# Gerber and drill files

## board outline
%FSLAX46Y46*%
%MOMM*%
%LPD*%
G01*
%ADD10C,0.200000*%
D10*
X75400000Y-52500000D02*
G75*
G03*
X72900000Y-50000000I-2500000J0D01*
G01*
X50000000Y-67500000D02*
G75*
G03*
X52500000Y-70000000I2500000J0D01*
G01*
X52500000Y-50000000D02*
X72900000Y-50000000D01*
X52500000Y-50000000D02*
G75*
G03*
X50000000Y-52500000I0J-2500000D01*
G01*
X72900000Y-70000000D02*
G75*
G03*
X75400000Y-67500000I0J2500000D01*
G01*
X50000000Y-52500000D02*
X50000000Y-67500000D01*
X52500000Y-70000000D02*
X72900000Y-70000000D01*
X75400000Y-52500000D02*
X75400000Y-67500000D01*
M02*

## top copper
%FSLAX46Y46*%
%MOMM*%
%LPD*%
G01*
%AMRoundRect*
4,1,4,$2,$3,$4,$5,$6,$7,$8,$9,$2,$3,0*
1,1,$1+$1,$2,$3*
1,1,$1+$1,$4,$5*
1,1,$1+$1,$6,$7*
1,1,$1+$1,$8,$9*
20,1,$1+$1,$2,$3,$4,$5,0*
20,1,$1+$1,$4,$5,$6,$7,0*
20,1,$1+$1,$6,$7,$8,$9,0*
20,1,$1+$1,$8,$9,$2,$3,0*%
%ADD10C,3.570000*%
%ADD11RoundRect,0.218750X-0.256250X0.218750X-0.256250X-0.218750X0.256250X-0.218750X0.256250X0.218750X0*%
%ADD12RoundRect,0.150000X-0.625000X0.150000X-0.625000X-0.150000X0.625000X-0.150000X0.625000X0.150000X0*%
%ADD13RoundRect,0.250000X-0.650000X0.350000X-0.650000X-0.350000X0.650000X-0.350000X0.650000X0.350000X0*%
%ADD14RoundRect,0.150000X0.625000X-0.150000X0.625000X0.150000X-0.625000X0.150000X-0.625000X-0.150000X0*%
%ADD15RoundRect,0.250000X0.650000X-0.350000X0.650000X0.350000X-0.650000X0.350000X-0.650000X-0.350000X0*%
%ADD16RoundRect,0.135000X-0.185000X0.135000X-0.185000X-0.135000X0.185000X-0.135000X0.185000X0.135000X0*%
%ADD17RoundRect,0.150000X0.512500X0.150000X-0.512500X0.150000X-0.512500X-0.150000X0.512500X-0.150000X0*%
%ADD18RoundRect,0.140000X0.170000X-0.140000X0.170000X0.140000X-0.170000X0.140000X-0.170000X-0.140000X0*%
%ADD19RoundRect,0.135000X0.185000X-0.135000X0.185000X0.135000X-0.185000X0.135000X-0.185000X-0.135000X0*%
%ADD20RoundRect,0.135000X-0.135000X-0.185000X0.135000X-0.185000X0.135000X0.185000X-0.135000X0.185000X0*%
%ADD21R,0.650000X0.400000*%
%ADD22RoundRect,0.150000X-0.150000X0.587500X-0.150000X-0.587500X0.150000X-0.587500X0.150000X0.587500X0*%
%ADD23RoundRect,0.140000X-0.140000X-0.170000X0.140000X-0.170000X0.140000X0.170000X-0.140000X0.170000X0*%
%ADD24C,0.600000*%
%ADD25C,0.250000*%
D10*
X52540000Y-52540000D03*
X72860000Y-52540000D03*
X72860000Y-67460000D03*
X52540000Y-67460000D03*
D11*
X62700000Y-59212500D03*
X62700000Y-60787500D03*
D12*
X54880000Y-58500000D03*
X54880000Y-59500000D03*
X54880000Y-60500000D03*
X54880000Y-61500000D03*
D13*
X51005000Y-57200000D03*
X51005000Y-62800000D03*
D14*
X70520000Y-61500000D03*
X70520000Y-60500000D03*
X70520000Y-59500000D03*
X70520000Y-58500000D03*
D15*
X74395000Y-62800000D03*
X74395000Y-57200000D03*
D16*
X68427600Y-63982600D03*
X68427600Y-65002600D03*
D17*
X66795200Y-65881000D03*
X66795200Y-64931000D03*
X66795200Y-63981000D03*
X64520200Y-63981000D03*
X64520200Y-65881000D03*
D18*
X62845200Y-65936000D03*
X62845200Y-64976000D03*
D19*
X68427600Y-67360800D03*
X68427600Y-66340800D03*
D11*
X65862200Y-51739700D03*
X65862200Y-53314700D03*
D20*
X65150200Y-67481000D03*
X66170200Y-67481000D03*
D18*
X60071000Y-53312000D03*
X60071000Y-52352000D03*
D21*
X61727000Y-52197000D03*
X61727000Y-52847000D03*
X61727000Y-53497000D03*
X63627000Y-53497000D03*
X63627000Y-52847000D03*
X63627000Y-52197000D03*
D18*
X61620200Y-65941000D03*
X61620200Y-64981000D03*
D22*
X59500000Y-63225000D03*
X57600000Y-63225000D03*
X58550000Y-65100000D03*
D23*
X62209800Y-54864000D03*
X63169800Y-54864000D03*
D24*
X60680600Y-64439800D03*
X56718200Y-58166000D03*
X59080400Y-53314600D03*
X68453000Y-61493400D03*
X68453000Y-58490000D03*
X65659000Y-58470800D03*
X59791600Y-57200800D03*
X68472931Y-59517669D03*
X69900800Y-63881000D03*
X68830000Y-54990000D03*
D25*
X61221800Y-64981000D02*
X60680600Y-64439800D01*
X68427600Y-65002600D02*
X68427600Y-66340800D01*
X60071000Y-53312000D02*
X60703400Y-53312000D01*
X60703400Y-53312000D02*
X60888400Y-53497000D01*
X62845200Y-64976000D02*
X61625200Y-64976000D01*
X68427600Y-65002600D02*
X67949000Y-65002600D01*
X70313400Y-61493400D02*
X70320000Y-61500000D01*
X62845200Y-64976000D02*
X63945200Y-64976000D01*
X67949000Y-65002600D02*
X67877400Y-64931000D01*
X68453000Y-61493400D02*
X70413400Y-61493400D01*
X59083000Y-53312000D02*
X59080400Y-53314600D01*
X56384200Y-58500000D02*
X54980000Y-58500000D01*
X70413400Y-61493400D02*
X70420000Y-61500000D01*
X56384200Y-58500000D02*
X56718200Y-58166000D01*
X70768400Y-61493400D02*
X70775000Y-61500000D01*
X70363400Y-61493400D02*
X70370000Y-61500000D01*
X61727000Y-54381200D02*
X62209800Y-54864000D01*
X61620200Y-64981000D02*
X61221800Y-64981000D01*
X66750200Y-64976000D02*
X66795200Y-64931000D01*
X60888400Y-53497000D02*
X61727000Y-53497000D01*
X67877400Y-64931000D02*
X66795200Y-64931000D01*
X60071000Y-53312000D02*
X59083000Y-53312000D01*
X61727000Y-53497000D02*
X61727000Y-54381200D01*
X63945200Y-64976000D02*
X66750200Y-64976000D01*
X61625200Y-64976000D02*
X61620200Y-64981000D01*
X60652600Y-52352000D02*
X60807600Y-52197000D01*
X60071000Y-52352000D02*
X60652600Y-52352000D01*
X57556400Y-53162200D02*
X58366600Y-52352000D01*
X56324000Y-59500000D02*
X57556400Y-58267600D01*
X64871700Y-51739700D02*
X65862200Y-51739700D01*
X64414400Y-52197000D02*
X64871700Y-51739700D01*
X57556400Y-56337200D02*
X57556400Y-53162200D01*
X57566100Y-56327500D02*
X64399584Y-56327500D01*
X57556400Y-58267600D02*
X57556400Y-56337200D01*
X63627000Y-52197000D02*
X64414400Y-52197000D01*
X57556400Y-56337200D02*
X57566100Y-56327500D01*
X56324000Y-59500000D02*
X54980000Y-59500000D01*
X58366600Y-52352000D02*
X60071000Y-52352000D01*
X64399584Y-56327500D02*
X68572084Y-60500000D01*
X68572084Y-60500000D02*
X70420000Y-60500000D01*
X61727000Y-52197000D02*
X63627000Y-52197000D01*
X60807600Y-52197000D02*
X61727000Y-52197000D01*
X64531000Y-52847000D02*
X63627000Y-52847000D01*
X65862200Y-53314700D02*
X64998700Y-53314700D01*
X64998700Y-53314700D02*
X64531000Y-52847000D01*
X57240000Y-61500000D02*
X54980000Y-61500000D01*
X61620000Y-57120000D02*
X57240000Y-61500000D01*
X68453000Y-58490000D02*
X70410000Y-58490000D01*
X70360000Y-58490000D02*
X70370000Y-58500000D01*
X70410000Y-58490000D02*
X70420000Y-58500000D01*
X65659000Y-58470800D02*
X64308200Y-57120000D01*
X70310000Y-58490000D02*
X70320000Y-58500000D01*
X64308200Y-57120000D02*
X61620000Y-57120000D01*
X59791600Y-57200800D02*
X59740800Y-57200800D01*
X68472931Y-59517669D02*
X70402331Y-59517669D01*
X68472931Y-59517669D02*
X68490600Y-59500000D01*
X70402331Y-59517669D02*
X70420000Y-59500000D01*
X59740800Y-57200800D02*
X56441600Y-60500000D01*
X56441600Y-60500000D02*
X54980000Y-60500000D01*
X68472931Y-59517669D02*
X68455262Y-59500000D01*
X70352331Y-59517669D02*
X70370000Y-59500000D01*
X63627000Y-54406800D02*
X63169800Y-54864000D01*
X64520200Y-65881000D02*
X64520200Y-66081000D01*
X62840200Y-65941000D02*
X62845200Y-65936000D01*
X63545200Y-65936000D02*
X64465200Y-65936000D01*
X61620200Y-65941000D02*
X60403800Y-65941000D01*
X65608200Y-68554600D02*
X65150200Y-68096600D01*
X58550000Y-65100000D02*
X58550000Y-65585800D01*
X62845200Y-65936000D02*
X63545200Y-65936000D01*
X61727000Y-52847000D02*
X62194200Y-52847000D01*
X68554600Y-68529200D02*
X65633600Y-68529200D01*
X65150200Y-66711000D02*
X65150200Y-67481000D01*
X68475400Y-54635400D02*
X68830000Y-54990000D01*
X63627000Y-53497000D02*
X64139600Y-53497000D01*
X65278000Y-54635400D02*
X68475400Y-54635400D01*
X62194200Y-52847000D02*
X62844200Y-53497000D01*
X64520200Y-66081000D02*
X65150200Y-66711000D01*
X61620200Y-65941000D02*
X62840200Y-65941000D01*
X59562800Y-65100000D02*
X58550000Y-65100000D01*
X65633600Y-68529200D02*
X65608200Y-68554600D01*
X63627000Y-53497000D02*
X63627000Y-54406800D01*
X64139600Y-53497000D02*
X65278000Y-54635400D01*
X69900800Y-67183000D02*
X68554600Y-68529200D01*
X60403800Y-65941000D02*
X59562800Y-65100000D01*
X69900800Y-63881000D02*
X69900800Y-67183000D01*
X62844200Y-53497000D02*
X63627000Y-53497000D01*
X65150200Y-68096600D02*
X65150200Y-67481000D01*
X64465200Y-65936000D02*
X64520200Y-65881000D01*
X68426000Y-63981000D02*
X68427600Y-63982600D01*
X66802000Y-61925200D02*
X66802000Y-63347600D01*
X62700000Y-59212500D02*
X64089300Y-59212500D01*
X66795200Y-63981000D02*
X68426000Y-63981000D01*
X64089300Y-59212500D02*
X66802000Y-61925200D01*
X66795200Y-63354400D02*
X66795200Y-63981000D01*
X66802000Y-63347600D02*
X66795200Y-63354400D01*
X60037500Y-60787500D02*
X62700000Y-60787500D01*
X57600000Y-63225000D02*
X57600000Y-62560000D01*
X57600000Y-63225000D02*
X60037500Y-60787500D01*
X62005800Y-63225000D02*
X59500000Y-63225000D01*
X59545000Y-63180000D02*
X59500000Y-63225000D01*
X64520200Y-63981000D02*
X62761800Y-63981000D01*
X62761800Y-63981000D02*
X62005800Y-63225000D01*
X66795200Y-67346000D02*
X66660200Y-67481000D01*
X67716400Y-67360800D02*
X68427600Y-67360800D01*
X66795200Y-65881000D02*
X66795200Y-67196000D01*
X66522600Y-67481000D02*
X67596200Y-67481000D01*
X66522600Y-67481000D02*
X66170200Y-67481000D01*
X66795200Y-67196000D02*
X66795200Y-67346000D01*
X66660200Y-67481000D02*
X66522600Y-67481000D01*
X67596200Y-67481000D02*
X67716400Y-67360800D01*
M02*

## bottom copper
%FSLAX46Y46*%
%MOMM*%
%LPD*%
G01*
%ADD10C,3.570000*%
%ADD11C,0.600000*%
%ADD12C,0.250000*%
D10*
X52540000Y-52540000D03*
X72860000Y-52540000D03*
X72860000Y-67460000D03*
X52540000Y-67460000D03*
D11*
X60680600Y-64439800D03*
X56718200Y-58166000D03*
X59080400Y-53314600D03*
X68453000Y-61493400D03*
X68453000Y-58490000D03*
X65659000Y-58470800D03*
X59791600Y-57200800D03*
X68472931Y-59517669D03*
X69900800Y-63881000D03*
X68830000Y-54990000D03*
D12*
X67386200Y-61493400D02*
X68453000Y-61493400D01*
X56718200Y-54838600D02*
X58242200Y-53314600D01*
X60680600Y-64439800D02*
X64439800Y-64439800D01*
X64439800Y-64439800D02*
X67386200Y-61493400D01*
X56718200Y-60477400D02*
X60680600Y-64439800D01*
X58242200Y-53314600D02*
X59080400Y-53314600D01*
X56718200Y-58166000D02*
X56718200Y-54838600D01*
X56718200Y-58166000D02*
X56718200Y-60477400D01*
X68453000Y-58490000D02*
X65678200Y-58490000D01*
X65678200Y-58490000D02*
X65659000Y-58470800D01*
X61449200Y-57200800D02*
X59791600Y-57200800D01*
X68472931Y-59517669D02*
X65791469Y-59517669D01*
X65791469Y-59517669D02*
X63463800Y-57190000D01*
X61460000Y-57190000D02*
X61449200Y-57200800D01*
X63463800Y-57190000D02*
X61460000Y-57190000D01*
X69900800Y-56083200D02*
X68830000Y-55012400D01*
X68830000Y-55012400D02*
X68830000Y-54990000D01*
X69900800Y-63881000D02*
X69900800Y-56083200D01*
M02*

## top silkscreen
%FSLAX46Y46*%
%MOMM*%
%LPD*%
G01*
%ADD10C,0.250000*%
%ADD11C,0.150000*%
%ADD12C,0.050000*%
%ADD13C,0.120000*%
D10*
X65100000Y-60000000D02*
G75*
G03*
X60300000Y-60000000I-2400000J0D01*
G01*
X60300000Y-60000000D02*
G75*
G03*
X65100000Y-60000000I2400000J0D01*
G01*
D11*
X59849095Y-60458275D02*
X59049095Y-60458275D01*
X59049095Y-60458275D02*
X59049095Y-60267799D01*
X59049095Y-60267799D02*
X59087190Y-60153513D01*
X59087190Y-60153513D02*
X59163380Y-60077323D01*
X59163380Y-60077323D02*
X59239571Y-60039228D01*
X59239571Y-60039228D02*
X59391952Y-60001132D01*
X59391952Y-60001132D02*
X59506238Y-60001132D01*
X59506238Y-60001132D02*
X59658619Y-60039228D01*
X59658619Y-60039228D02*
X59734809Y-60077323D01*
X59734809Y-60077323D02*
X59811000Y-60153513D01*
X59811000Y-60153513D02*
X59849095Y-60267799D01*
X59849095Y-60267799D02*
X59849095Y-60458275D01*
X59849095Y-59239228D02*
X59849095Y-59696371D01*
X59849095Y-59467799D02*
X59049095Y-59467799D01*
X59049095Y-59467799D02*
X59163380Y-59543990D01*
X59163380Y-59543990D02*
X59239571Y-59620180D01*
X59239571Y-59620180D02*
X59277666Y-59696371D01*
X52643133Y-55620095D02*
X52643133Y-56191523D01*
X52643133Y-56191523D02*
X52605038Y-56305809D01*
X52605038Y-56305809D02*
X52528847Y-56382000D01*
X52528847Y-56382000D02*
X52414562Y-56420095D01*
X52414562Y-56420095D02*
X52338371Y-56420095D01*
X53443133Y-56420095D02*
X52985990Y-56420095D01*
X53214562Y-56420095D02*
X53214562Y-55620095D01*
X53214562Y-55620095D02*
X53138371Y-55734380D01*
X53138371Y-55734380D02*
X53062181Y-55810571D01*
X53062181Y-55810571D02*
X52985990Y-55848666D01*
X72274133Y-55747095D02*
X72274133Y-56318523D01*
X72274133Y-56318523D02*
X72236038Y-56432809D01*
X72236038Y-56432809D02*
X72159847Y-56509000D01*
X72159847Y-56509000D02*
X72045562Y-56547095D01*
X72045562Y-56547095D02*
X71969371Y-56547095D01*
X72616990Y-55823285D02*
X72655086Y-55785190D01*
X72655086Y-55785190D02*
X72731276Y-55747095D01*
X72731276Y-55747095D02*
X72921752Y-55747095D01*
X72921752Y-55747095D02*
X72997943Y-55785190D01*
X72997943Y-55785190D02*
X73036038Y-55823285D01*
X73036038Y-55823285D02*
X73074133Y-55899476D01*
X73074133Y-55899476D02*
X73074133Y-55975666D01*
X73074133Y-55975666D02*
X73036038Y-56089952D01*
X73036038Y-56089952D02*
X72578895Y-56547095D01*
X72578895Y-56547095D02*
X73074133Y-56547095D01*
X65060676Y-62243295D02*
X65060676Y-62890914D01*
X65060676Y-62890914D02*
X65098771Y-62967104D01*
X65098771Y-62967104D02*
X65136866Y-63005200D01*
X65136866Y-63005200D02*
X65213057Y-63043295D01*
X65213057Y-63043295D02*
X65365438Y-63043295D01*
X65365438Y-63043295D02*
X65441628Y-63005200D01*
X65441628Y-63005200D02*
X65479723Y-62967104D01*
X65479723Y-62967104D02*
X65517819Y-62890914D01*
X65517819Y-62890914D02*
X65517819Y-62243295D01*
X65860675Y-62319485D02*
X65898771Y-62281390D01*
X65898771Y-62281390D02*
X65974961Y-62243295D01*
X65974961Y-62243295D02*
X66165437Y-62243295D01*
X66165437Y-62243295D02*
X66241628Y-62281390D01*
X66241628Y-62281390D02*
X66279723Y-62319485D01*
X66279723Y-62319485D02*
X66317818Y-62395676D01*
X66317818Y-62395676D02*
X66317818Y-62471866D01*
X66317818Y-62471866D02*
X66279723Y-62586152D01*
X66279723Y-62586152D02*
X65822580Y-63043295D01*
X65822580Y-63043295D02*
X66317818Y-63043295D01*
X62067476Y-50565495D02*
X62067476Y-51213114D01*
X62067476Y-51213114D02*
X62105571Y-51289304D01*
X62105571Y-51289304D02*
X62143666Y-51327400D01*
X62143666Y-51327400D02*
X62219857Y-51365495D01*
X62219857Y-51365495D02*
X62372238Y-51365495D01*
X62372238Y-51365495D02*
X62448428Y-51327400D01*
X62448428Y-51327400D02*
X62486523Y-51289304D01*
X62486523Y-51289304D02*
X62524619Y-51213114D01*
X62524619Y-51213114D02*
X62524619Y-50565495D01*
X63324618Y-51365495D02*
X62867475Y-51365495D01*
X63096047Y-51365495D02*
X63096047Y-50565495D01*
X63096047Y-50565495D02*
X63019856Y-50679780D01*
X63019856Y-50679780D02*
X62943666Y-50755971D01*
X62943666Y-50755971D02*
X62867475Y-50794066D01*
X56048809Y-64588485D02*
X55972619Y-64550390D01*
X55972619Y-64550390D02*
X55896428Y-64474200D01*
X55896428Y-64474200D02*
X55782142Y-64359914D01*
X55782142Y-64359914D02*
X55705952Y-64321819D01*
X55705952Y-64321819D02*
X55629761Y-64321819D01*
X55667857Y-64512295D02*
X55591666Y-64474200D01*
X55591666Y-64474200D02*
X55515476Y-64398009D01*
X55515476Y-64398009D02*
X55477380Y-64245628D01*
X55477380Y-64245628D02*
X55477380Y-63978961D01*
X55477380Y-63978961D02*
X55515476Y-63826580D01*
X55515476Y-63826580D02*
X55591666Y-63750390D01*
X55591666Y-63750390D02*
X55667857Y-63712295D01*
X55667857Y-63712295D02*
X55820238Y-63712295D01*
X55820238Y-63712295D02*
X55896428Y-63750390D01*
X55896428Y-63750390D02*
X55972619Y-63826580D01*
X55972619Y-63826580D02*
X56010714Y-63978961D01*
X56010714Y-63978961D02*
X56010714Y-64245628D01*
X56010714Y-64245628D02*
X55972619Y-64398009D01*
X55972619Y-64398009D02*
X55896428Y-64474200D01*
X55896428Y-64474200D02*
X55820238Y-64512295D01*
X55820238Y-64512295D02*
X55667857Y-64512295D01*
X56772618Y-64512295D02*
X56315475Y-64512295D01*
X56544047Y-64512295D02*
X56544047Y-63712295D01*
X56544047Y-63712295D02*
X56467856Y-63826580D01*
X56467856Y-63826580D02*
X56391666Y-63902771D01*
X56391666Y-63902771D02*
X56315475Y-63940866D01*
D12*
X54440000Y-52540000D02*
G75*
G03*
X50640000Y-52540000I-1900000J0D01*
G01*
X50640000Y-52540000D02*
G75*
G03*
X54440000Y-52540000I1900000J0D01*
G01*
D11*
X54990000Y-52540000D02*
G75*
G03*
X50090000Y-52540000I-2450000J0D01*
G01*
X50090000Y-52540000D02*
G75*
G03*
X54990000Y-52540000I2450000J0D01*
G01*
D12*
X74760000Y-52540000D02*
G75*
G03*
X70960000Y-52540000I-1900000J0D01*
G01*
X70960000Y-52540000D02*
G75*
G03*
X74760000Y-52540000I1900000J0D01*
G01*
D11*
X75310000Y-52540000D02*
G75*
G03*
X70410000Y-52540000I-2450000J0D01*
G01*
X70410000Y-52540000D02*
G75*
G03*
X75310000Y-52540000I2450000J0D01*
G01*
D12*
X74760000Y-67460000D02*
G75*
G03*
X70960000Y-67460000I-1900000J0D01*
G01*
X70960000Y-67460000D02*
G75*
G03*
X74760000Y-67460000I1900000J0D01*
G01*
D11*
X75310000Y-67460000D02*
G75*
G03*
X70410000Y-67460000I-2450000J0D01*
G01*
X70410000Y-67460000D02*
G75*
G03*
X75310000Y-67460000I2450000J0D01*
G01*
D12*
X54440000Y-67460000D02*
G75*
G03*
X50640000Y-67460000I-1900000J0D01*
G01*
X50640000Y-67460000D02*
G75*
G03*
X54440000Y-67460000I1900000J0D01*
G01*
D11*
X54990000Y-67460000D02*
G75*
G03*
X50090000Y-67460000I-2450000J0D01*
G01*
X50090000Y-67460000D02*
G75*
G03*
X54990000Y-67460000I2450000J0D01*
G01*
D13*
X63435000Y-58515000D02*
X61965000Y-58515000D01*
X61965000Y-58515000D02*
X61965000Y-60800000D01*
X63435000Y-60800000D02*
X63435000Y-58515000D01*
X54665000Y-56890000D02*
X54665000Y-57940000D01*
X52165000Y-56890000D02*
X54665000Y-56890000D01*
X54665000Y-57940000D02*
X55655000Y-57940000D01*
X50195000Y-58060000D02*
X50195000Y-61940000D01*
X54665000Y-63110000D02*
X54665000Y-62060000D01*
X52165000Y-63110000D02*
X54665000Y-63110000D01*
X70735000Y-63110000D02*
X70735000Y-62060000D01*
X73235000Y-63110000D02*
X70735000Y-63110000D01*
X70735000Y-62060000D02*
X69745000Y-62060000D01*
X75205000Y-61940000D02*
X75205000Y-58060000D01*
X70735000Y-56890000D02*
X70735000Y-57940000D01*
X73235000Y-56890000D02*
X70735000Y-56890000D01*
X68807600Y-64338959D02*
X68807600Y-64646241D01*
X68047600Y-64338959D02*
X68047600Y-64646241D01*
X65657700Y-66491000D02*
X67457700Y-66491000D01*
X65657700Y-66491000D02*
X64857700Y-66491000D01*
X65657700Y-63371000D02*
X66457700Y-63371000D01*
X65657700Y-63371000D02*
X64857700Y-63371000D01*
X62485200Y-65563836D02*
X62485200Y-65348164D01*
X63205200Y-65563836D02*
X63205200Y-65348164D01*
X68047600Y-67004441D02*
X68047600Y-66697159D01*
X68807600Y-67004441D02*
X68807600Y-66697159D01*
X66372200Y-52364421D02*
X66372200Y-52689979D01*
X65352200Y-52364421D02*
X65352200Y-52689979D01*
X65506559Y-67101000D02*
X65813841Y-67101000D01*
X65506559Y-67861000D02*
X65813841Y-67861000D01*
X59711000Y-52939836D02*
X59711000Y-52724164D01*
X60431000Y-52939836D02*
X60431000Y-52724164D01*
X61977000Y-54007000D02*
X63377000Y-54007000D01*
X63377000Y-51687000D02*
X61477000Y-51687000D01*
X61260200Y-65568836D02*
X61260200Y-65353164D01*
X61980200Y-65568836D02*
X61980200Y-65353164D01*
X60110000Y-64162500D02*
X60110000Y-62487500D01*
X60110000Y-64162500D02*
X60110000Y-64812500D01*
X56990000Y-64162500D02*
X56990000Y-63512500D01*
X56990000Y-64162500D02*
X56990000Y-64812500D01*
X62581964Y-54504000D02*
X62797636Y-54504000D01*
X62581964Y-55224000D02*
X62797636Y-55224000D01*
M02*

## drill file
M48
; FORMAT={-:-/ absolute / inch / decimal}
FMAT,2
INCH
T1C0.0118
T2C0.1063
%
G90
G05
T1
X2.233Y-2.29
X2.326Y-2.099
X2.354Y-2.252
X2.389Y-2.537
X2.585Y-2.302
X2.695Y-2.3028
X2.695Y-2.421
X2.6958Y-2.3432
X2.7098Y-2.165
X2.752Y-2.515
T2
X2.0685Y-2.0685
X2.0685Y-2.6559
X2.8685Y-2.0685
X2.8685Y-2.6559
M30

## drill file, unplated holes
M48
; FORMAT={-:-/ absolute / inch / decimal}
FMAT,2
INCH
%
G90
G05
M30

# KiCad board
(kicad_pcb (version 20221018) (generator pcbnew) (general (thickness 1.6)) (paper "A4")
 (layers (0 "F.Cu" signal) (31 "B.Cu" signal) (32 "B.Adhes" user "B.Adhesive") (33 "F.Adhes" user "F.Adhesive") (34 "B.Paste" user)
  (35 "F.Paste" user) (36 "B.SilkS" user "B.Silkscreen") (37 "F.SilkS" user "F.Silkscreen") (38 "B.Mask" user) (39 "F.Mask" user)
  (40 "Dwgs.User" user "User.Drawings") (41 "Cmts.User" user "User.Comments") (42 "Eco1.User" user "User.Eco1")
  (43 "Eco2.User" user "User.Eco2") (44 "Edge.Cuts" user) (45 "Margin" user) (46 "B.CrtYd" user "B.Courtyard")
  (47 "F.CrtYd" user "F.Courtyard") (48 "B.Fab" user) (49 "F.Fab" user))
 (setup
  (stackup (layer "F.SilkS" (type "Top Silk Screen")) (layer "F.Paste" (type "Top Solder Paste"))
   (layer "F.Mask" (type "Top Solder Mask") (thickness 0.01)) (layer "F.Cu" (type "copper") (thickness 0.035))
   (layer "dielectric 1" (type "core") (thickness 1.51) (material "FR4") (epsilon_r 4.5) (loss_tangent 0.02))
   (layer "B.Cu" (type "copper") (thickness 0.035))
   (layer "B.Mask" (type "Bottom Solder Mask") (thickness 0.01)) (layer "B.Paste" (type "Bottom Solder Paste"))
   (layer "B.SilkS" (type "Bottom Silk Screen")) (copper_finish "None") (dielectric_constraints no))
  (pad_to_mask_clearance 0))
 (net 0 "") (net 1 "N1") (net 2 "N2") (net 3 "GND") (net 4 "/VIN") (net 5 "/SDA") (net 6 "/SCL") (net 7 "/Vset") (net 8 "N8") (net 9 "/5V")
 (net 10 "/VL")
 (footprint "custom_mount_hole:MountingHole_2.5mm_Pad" (layer "F.Cu") (at 52.54 52.54)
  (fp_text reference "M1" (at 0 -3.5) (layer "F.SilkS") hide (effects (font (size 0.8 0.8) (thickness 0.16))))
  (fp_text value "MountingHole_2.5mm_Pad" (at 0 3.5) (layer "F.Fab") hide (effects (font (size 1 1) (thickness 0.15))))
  (fp_circle (center 0 0) (end 1.9 0) (stroke (width 0.05) (type solid)) (fill none) (layer "F.SilkS"))
  (fp_circle (center 0 0) (end 2.45 0) (stroke (width 0.15) (type solid)) (fill none) (layer "F.SilkS"))
  (pad "~" thru_hole circle (at 0 0) (size 3.57 3.57) (drill 2.7) (layers "*.Cu" "*.Mask")))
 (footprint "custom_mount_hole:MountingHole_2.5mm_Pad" (layer "F.Cu") (at 72.86 52.54)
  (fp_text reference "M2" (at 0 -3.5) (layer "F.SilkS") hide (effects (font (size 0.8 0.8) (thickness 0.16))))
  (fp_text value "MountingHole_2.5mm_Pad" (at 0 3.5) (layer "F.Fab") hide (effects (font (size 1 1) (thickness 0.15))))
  (fp_circle (center 0 0) (end 1.9 0) (stroke (width 0.05) (type solid)) (fill none) (layer "F.SilkS"))
  (fp_circle (center 0 0) (end 2.45 0) (stroke (width 0.15) (type solid)) (fill none) (layer "F.SilkS"))
  (pad "~" thru_hole circle (at 0 0) (size 3.57 3.57) (drill 2.7) (layers "*.Cu" "*.Mask")))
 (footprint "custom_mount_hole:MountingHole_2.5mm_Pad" (layer "F.Cu") (at 72.86 67.46)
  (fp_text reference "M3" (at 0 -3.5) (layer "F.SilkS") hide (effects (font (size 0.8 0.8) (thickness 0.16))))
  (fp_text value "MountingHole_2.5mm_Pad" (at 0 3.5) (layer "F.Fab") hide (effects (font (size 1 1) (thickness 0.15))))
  (fp_circle (center 0 0) (end 1.9 0) (stroke (width 0.05) (type solid)) (fill none) (layer "F.SilkS"))
  (fp_circle (center 0 0) (end 2.45 0) (stroke (width 0.15) (type solid)) (fill none) (layer "F.SilkS"))
  (pad "~" thru_hole circle (at 0 0) (size 3.57 3.57) (drill 2.7) (layers "*.Cu" "*.Mask")))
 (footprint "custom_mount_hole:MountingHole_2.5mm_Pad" (layer "F.Cu") (at 52.54 67.46)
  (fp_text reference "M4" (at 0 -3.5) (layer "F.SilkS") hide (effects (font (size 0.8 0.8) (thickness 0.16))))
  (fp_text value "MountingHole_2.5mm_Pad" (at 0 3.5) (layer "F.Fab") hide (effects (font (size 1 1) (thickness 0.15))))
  (fp_circle (center 0 0) (end 1.9 0) (stroke (width 0.05) (type solid)) (fill none) (layer "F.SilkS"))
  (fp_circle (center 0 0) (end 2.45 0) (stroke (width 0.15) (type solid)) (fill none) (layer "F.SilkS"))
  (pad "~" thru_hole circle (at 0 0) (size 3.57 3.57) (drill 2.7) (layers "*.Cu" "*.Mask")))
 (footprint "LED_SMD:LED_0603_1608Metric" (layer "F.Cu") (at 62.7 60 -90)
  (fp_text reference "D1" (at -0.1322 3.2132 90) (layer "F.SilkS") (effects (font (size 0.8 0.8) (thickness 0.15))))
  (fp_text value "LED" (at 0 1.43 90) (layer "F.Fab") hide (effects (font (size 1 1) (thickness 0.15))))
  (fp_line (start -1.485 -0.735) (end -1.485 0.735) (stroke (width 0.12) (type solid)) (layer "F.SilkS"))
  (fp_line (start -1.485 0.735) (end 0.8 0.735) (stroke (width 0.12) (type solid)) (layer "F.SilkS"))
  (fp_line (start 0.8 -0.735) (end -1.485 -0.735) (stroke (width 0.12) (type solid)) (layer "F.SilkS"))
  (pad "1" smd roundrect (at -0.7875 0 270) (size 0.875 0.95) (layers "F.Cu" "F.Paste" "F.Mask") (roundrect_rratio 0.25) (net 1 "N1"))
  (pad "2" smd roundrect (at 0.7875 0 270) (size 0.875 0.95) (layers "F.Cu" "F.Paste" "F.Mask") (roundrect_rratio 0.25) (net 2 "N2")))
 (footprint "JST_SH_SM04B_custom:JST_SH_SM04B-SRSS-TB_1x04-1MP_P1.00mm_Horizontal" (layer "F.Cu") (at 52.88 60 -90)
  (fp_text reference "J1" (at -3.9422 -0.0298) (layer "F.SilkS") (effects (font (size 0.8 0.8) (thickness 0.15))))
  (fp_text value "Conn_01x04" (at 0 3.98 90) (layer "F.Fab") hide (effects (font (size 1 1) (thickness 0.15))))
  (fp_line (start -3.11 -1.785) (end -2.06 -1.785) (stroke (width 0.12) (type solid)) (layer "F.SilkS"))
  (fp_line (start -3.11 0.715) (end -3.11 -1.785) (stroke (width 0.12) (type solid)) (layer "F.SilkS"))
  (fp_line (start -2.06 -1.785) (end -2.06 -2.775) (stroke (width 0.12) (type solid)) (layer "F.SilkS"))
  (fp_line (start -1.94 2.685) (end 1.94 2.685) (stroke (width 0.12) (type solid)) (layer "F.SilkS"))
  (fp_line (start 3.11 -1.785) (end 2.06 -1.785) (stroke (width 0.12) (type solid)) (layer "F.SilkS"))
  (fp_line (start 3.11 0.715) (end 3.11 -1.785) (stroke (width 0.12) (type solid)) (layer "F.SilkS"))
  (pad "1" smd roundrect (at -1.5 -2 270) (size 0.6 1.55) (layers "F.Cu" "F.Paste" "F.Mask") (roundrect_rratio 0.25) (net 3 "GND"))
  (pad "2" smd roundrect (at -0.5 -2 270) (size 0.6 1.55) (layers "F.Cu" "F.Paste" "F.Mask") (roundrect_rratio 0.25) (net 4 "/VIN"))
  (pad "3" smd roundrect (at 0.5 -2 270) (size 0.6 1.55) (layers "F.Cu" "F.Paste" "F.Mask") (roundrect_rratio 0.25) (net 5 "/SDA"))
  (pad "4" smd roundrect (at 1.5 -2 270) (size 0.6 1.55) (layers "F.Cu" "F.Paste" "F.Mask") (roundrect_rratio 0.25) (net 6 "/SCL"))
  (pad "MP" smd roundrect (at -2.8 1.875 270) (size 1.2 1.8) (layers "F.Cu" "F.Paste" "F.Mask") (roundrect_rratio 0.2083333333))
  (pad "MP" smd roundrect (at 2.8 1.875 270) (size 1.2 1.8) (layers "F.Cu" "F.Paste" "F.Mask") (roundrect_rratio 0.2083333333)))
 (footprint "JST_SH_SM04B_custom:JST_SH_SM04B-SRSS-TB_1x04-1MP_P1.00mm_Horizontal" (layer "F.Cu") (at 72.52 60 90)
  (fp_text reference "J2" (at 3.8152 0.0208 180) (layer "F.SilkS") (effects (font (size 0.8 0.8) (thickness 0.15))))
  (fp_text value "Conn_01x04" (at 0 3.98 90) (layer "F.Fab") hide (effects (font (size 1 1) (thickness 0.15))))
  (fp_line (start -3.11 -1.785) (end -2.06 -1.785) (stroke (width 0.12) (type solid)) (layer "F.SilkS"))
  (fp_line (start -3.11 0.715) (end -3.11 -1.785) (stroke (width 0.12) (type solid)) (layer "F.SilkS"))
  (fp_line (start -2.06 -1.785) (end -2.06 -2.775) (stroke (width 0.12) (type solid)) (layer "F.SilkS"))
  (fp_line (start -1.94 2.685) (end 1.94 2.685) (stroke (width 0.12) (type solid)) (layer "F.SilkS"))
  (fp_line (start 3.11 -1.785) (end 2.06 -1.785) (stroke (width 0.12) (type solid)) (layer "F.SilkS"))
  (fp_line (start 3.11 0.715) (end 3.11 -1.785) (stroke (width 0.12) (type solid)) (layer "F.SilkS"))
  (pad "1" smd roundrect (at -1.5 -2 90) (size 0.6 1.55) (layers "F.Cu" "F.Paste" "F.Mask") (roundrect_rratio 0.25) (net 3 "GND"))
  (pad "2" smd roundrect (at -0.5 -2 90) (size 0.6 1.55) (layers "F.Cu" "F.Paste" "F.Mask") (roundrect_rratio 0.25) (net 4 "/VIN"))
  (pad "3" smd roundrect (at 0.5 -2 90) (size 0.6 1.55) (layers "F.Cu" "F.Paste" "F.Mask") (roundrect_rratio 0.25) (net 5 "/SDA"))
  (pad "4" smd roundrect (at 1.5 -2 90) (size 0.6 1.55) (layers "F.Cu" "F.Paste" "F.Mask") (roundrect_rratio 0.25) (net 6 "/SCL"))
  (pad "MP" smd roundrect (at -2.8 1.875 90) (size 1.2 1.8) (layers "F.Cu" "F.Paste" "F.Mask") (roundrect_rratio 0.2083333333))
  (pad "MP" smd roundrect (at 2.8 1.875 90) (size 1.2 1.8) (layers "F.Cu" "F.Paste" "F.Mask") (roundrect_rratio 0.2083333333)))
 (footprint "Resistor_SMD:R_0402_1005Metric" (layer "F.Cu") (at 68.4276 64.4926 -90)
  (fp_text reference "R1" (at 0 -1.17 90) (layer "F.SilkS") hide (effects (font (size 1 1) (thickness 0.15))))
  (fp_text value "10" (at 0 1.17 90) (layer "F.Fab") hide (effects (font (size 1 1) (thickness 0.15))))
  (fp_line (start -0.153641 -0.38) (end 0.153641 -0.38) (stroke (width 0.12) (type solid)) (layer "F.SilkS"))
  (fp_line (start -0.153641 0.38) (end 0.153641 0.38) (stroke (width 0.12) (type solid)) (layer "F.SilkS"))
  (pad "1" smd roundrect (at -0.51 0 270) (size 0.54 0.64) (layers "F.Cu" "F.Paste" "F.Mask") (roundrect_rratio 0.25) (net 1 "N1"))
  (pad "2" smd roundrect (at 0.51 0 270) (size 0.54 0.64) (layers "F.Cu" "F.Paste" "F.Mask") (roundrect_rratio 0.25) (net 3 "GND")))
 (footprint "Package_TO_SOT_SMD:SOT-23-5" (layer "F.Cu") (at 65.6577 64.931 180)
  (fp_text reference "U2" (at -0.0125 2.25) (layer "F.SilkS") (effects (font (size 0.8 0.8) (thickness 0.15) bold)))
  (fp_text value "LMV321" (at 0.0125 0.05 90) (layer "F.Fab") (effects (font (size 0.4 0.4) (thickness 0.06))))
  (fp_line (start 0 -1.56) (end -1.8 -1.56) (stroke (width 0.12) (type solid)) (layer "F.SilkS"))
  (fp_line (start 0 -1.56) (end 0.8 -1.56) (stroke (width 0.12) (type solid)) (layer "F.SilkS"))
  (fp_line (start 0 1.56) (end -0.8 1.56) (stroke (width 0.12) (type solid)) (layer "F.SilkS"))
  (fp_line (start 0 1.56) (end 0.8 1.56) (stroke (width 0.12) (type solid)) (layer "F.SilkS"))
  (pad "1" smd roundrect (at -1.1375 -0.95 180) (size 1.325 0.6) (layers "F.Cu" "F.Paste" "F.Mask") (roundrect_rratio 0.25) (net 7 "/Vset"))
  (pad "2" smd roundrect (at -1.1375 0 180) (size 1.325 0.6) (layers "F.Cu" "F.Paste" "F.Mask") (roundrect_rratio 0.25) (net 3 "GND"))
  (pad "3" smd roundrect (at -1.1375 0.95 180) (size 1.325 0.6) (layers "F.Cu" "F.Paste" "F.Mask") (roundrect_rratio 0.25) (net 1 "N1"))
  (pad "4" smd roundrect (at 1.1375 0.95 180) (size 1.325 0.6) (layers "F.Cu" "F.Paste" "F.Mask") (roundrect_rratio 0.25) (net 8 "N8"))
  (pad "5" smd roundrect (at 1.1375 -0.95 180) (size 1.325 0.6) (layers "F.Cu" "F.Paste" "F.Mask") (roundrect_rratio 0.25) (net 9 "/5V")))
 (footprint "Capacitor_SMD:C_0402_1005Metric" (layer "F.Cu") (at 62.8452 65.456 90)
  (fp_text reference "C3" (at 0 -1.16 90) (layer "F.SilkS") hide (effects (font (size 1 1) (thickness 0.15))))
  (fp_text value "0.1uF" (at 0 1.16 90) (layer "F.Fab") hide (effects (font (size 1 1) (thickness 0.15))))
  (fp_line (start -0.107836 -0.36) (end 0.107836 -0.36) (stroke (width 0.12) (type solid)) (layer "F.SilkS"))
  (fp_line (start -0.107836 0.36) (end 0.107836 0.36) (stroke (width 0.12) (type solid)) (layer "F.SilkS"))
  (pad "1" smd roundrect (at -0.48 0 90) (size 0.56 0.62) (layers "F.Cu" "F.Paste" "F.Mask") (roundrect_rratio 0.25) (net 9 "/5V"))
  (pad "2" smd roundrect (at 0.48 0 90) (size 0.56 0.62) (layers "F.Cu" "F.Paste" "F.Mask") (roundrect_rratio 0.25) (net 3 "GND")))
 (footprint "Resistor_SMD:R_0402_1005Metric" (layer "F.Cu") (at 68.4276 66.8508 90)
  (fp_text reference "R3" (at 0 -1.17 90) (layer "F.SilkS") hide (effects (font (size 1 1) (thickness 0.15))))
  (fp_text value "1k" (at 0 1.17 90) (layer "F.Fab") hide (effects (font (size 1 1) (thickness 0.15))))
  (fp_line (start -0.153641 -0.38) (end 0.153641 -0.38) (stroke (width 0.12) (type solid)) (layer "F.SilkS"))
  (fp_line (start -0.153641 0.38) (end 0.153641 0.38) (stroke (width 0.12) (type solid)) (layer "F.SilkS"))
  (pad "1" smd roundrect (at -0.51 0 90) (size 0.54 0.64) (layers "F.Cu" "F.Paste" "F.Mask") (roundrect_rratio 0.25) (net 7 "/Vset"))
  (pad "2" smd roundrect (at 0.51 0 90) (size 0.54 0.64) (layers "F.Cu" "F.Paste" "F.Mask") (roundrect_rratio 0.25) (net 3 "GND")))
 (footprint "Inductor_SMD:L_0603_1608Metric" (layer "F.Cu") (at 65.8622 52.5272 -90)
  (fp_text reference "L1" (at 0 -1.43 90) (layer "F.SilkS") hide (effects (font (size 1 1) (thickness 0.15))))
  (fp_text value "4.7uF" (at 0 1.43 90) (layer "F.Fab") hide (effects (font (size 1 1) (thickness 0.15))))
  (fp_line (start -0.162779 -0.51) (end 0.162779 -0.51) (stroke (width 0.12) (type solid)) (layer "F.SilkS"))
  (fp_line (start -0.162779 0.51) (end 0.162779 0.51) (stroke (width 0.12) (type solid)) (layer "F.SilkS"))
  (pad "1" smd roundrect (at -0.7875 0 270) (size 0.875 0.95) (layers "F.Cu" "F.Paste" "F.Mask") (roundrect_rratio 0.25) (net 4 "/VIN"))
  (pad "2" smd roundrect (at 0.7875 0 270) (size 0.875 0.95) (layers "F.Cu" "F.Paste" "F.Mask") (roundrect_rratio 0.25) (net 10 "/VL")))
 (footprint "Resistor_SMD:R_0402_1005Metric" (layer "F.Cu") (at 65.6602 67.481)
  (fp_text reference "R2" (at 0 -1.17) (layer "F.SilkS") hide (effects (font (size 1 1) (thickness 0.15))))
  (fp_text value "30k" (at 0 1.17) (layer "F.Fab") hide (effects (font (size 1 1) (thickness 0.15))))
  (fp_line (start -0.153641 -0.38) (end 0.153641 -0.38) (stroke (width 0.12) (type solid)) (layer "F.SilkS"))
  (fp_line (start -0.153641 0.38) (end 0.153641 0.38) (stroke (width 0.12) (type solid)) (layer "F.SilkS"))
  (pad "1" smd roundrect (at -0.51 0) (size 0.54 0.64) (layers "F.Cu" "F.Paste" "F.Mask") (roundrect_rratio 0.25) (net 9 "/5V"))
  (pad "2" smd roundrect (at 0.51 0) (size 0.54 0.64) (layers "F.Cu" "F.Paste" "F.Mask") (roundrect_rratio 0.25) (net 7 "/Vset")))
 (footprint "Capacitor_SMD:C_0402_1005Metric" (layer "F.Cu") (at 60.071 52.832 90)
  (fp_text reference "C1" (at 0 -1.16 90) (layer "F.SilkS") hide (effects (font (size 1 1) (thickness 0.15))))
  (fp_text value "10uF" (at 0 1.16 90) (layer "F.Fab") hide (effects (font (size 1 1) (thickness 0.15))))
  (fp_line (start -0.107836 -0.36) (end 0.107836 -0.36) (stroke (width 0.12) (type solid)) (layer "F.SilkS"))
  (fp_line (start -0.107836 0.36) (end 0.107836 0.36) (stroke (width 0.12) (type solid)) (layer "F.SilkS"))
  (pad "1" smd roundrect (at -0.48 0 90) (size 0.56 0.62) (layers "F.Cu" "F.Paste" "F.Mask") (roundrect_rratio 0.25) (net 3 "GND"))
  (pad "2" smd roundrect (at 0.48 0 90) (size 0.56 0.62) (layers "F.Cu" "F.Paste" "F.Mask") (roundrect_rratio 0.25) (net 4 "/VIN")))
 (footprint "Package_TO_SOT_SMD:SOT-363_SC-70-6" (layer "F.Cu") (at 62.677 52.847)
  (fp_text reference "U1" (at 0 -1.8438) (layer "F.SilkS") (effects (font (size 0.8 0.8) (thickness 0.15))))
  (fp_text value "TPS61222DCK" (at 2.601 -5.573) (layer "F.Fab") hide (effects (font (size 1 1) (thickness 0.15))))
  (fp_line (start -0.7 1.16) (end 0.7 1.16) (stroke (width 0.12) (type solid)) (layer "F.SilkS"))
  (fp_line (start 0.7 -1.16) (end -1.2 -1.16) (stroke (width 0.12) (type solid)) (layer "F.SilkS"))
  (pad "1" smd rect (at -0.95 -0.65) (size 0.65 0.4) (layers "F.Cu" "F.Paste" "F.Mask") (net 4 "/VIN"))
  (pad "2" smd rect (at -0.95 0) (size 0.65 0.4) (layers "F.Cu" "F.Paste" "F.Mask") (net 9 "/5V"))
  (pad "3" smd rect (at -0.95 0.65) (size 0.65 0.4) (layers "F.Cu" "F.Paste" "F.Mask") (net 3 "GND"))
  (pad "4" smd rect (at 0.95 0.65) (size 0.65 0.4) (layers "F.Cu" "F.Paste" "F.Mask") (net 9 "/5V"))
  (pad "5" smd rect (at 0.95 0) (size 0.65 0.4) (layers "F.Cu" "F.Paste" "F.Mask") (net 10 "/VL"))
  (pad "6" smd rect (at 0.95 -0.65) (size 0.65 0.4) (layers "F.Cu" "F.Paste" "F.Mask") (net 4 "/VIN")))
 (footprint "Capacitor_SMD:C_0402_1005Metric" (layer "F.Cu") (at 61.6202 65.461 90)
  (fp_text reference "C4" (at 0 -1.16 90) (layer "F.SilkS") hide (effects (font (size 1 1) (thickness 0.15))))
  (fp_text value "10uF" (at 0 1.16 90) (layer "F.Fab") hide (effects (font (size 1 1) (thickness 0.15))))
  (fp_line (start -0.107836 -0.36) (end 0.107836 -0.36) (stroke (width 0.12) (type solid)) (layer "F.SilkS"))
  (fp_line (start -0.107836 0.36) (end 0.107836 0.36) (stroke (width 0.12) (type solid)) (layer "F.SilkS"))
  (pad "1" smd roundrect (at -0.48 0 90) (size 0.56 0.62) (layers "F.Cu" "F.Paste" "F.Mask") (roundrect_rratio 0.25) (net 9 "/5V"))
  (pad "2" smd roundrect (at 0.48 0 90) (size 0.56 0.62) (layers "F.Cu" "F.Paste" "F.Mask") (roundrect_rratio 0.25) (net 3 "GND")))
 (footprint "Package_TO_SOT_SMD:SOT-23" (layer "F.Cu") (at 58.55 64.1625 -90)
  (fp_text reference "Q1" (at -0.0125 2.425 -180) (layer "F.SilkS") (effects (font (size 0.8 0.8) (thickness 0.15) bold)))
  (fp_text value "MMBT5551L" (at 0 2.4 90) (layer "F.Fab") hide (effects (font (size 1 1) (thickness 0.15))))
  (fp_line (start 0 -1.56) (end -1.675 -1.56) (stroke (width 0.12) (type solid)) (layer "F.SilkS"))
  (fp_line (start 0 -1.56) (end 0.65 -1.56) (stroke (width 0.12) (type solid)) (layer "F.SilkS"))
  (fp_line (start 0 1.56) (end -0.65 1.56) (stroke (width 0.12) (type solid)) (layer "F.SilkS"))
  (fp_line (start 0 1.56) (end 0.65 1.56) (stroke (width 0.12) (type solid)) (layer "F.SilkS"))
  (pad "1" smd roundrect (at -0.9375 -0.95 270) (size 1.475 0.6) (layers "F.Cu" "F.Paste" "F.Mask") (roundrect_rratio 0.25) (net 8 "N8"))
  (pad "2" smd roundrect (at -0.9375 0.95 270) (size 1.475 0.6) (layers "F.Cu" "F.Paste" "F.Mask") (roundrect_rratio 0.25) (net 2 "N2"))
  (pad "3" smd roundrect (at 0.9375 0 270) (size 1.475 0.6) (layers "F.Cu" "F.Paste" "F.Mask") (roundrect_rratio 0.25) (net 9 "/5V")))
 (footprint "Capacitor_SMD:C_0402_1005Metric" (layer "F.Cu") (at 62.6898 54.864)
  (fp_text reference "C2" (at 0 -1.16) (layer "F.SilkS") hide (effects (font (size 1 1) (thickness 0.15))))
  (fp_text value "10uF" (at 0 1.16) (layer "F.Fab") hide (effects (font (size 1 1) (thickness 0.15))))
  (fp_line (start -0.107836 -0.36) (end 0.107836 -0.36) (stroke (width 0.12) (type solid)) (layer "F.SilkS"))
  (fp_line (start -0.107836 0.36) (end 0.107836 0.36) (stroke (width 0.12) (type solid)) (layer "F.SilkS"))
  (pad "1" smd roundrect (at -0.48 0) (size 0.56 0.62) (layers "F.Cu" "F.Paste" "F.Mask") (roundrect_rratio 0.25) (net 3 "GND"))
  (pad "2" smd roundrect (at 0.48 0) (size 0.56 0.62) (layers "F.Cu" "F.Paste" "F.Mask") (roundrect_rratio 0.25) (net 9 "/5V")))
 (gr_circle (center 62.7 60) (end 65.1 60) (stroke (width 0.25) (type solid)) (fill none) (layer "F.SilkS"))
 (gr_arc (start 72.9 50) (mid 74.667767 50.732233) (end 75.4 52.5) (stroke (width 0.2) (type solid)) (layer "Edge.Cuts"))
 (gr_arc (start 52.5 70) (mid 50.732233 69.267767) (end 50 67.5) (stroke (width 0.2) (type solid)) (layer "Edge.Cuts"))
 (gr_line (start 52.5 50) (end 72.9 50) (stroke (width 0.2) (type solid)) (layer "Edge.Cuts"))
 (gr_arc (start 50 52.5) (mid 50.732233 50.732233) (end 52.5 50) (stroke (width 0.2) (type solid)) (layer "Edge.Cuts"))
 (gr_arc (start 75.4 67.5) (mid 74.667767 69.267767) (end 72.9 70) (stroke (width 0.2) (type solid)) (layer "Edge.Cuts"))
 (gr_line (start 50 52.5) (end 50 67.5) (stroke (width 0.2) (type solid)) (layer "Edge.Cuts"))
 (gr_line (start 52.5 70) (end 72.9 70) (stroke (width 0.2) (type solid)) (layer "Edge.Cuts"))
 (gr_line (start 75.4 52.5) (end 75.4 67.5) (stroke (width 0.2) (type solid)) (layer "Edge.Cuts"))
 (segment (start 61.2218 64.981) (end 60.6806 64.4398) (width 0.25) (layer "F.Cu") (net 3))
 (segment (start 68.4276 65.0026) (end 68.4276 66.3408) (width 0.25) (layer "F.Cu") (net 3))
 (segment (start 60.071 53.312) (end 60.7034 53.312) (width 0.25) (layer "F.Cu") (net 3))
 (segment (start 60.7034 53.312) (end 60.8884 53.497) (width 0.25) (layer "F.Cu") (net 3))
 (segment (start 62.8452 64.976) (end 61.6252 64.976) (width 0.25) (layer "F.Cu") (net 3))
 (segment (start 68.4276 65.0026) (end 67.949 65.0026) (width 0.25) (layer "F.Cu") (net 3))
 (segment (start 70.3134 61.4934) (end 70.32 61.5) (width 0.25) (layer "F.Cu") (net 3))
 (segment (start 62.8452 64.976) (end 63.9452 64.976) (width 0.25) (layer "F.Cu") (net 3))
 (segment (start 67.949 65.0026) (end 67.8774 64.931) (width 0.25) (layer "F.Cu") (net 3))
 (segment (start 68.453 61.4934) (end 70.4134 61.4934) (width 0.25) (layer "F.Cu") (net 3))
 (segment (start 59.083 53.312) (end 59.0804 53.3146) (width 0.25) (layer "F.Cu") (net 3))
 (segment (start 56.3842 58.5) (end 54.98 58.5) (width 0.25) (layer "F.Cu") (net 3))
 (segment (start 70.4134 61.4934) (end 70.42 61.5) (width 0.25) (layer "F.Cu") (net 3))
 (segment (start 56.3842 58.5) (end 56.7182 58.166) (width 0.25) (layer "F.Cu") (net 3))
 (segment (start 70.7684 61.4934) (end 70.775 61.5) (width 0.25) (layer "F.Cu") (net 3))
 (segment (start 70.3634 61.4934) (end 70.37 61.5) (width 0.25) (layer "F.Cu") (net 3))
 (segment (start 61.727 54.3812) (end 62.2098 54.864) (width 0.25) (layer "F.Cu") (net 3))
 (segment (start 61.6202 64.981) (end 61.2218 64.981) (width 0.25) (layer "F.Cu") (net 3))
 (segment (start 66.7502 64.976) (end 66.7952 64.931) (width 0.25) (layer "F.Cu") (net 3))
 (segment (start 60.8884 53.497) (end 61.727 53.497) (width 0.25) (layer "F.Cu") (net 3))
 (segment (start 67.8774 64.931) (end 66.7952 64.931) (width 0.25) (layer "F.Cu") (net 3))
 (segment (start 60.071 53.312) (end 59.083 53.312) (width 0.25) (layer "F.Cu") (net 3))
 (segment (start 61.727 53.497) (end 61.727 54.3812) (width 0.25) (layer "F.Cu") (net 3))
 (segment (start 63.9452 64.976) (end 66.7502 64.976) (width 0.25) (layer "F.Cu") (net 3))
 (segment (start 61.6252 64.976) (end 61.6202 64.981) (width 0.25) (layer "F.Cu") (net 3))
 (via (at 60.6806 64.4398) (size 0.6) (drill 0.3) (layers "F.Cu" "B.Cu") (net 3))
 (via (at 56.7182 58.166) (size 0.6) (drill 0.3) (layers "F.Cu" "B.Cu") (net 3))
 (via (at 59.0804 53.3146) (size 0.6) (drill 0.3) (layers "F.Cu" "B.Cu") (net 3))
 (via (at 68.453 61.4934) (size 0.6) (drill 0.3) (layers "F.Cu" "B.Cu") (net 3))
 (segment (start 67.3862 61.4934) (end 68.453 61.4934) (width 0.25) (layer "B.Cu") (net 3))
 (segment (start 56.7182 54.8386) (end 58.2422 53.3146) (width 0.25) (layer "B.Cu") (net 3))
 (segment (start 60.6806 64.4398) (end 64.4398 64.4398) (width 0.25) (layer "B.Cu") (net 3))
 (segment (start 64.4398 64.4398) (end 67.3862 61.4934) (width 0.25) (layer "B.Cu") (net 3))
 (segment (start 56.7182 60.4774) (end 60.6806 64.4398) (width 0.25) (layer "B.Cu") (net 3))
 (segment (start 58.2422 53.3146) (end 59.0804 53.3146) (width 0.25) (layer "B.Cu") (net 3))
 (segment (start 56.7182 58.166) (end 56.7182 54.8386) (width 0.25) (layer "B.Cu") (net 3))
 (segment (start 56.7182 58.166) (end 56.7182 60.4774) (width 0.25) (layer "B.Cu") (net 3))
 (segment (start 60.6526 52.352) (end 60.8076 52.197) (width 0.25) (layer "F.Cu") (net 4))
 (segment (start 60.071 52.352) (end 60.6526 52.352) (width 0.25) (layer "F.Cu") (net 4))
 (segment (start 57.5564 53.1622) (end 58.3666 52.352) (width 0.25) (layer "F.Cu") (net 4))
 (segment (start 56.324 59.5) (end 57.5564 58.2676) (width 0.25) (layer "F.Cu") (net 4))
 (segment (start 64.8717 51.7397) (end 65.8622 51.7397) (width 0.25) (layer "F.Cu") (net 4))
 (segment (start 64.4144 52.197) (end 64.8717 51.7397) (width 0.25) (layer "F.Cu") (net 4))
 (segment (start 57.5564 56.3372) (end 57.5564 53.1622) (width 0.25) (layer "F.Cu") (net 4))
 (segment (start 57.5661 56.3275) (end 64.399584 56.3275) (width 0.25) (layer "F.Cu") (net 4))
 (segment (start 57.5564 58.2676) (end 57.5564 56.3372) (width 0.25) (layer "F.Cu") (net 4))
 (segment (start 63.627 52.197) (end 64.4144 52.197) (width 0.25) (layer "F.Cu") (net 4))
 (segment (start 57.5564 56.3372) (end 57.5661 56.3275) (width 0.25) (layer "F.Cu") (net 4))
 (segment (start 56.324 59.5) (end 54.98 59.5) (width 0.25) (layer "F.Cu") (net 4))
 (segment (start 58.3666 52.352) (end 60.071 52.352) (width 0.25) (layer "F.Cu") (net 4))
 (segment (start 64.399584 56.3275) (end 68.572084 60.5) (width 0.25) (layer "F.Cu") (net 4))
 (segment (start 68.572084 60.5) (end 70.42 60.5) (width 0.25) (layer "F.Cu") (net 4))
 (segment (start 61.727 52.197) (end 63.627 52.197) (width 0.25) (layer "F.Cu") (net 4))
 (segment (start 60.8076 52.197) (end 61.727 52.197) (width 0.25) (layer "F.Cu") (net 4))
 (segment (start 64.531 52.847) (end 63.627 52.847) (width 0.25) (layer "F.Cu") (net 10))
 (segment (start 65.8622 53.3147) (end 64.9987 53.3147) (width 0.25) (layer "F.Cu") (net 10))
 (segment (start 64.9987 53.3147) (end 64.531 52.847) (width 0.25) (layer "F.Cu") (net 10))
 (segment (start 57.24 61.5) (end 54.98 61.5) (width 0.25) (layer "F.Cu") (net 6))
 (segment (start 61.62 57.12) (end 57.24 61.5) (width 0.25) (layer "F.Cu") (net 6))
 (segment (start 68.453 58.49) (end 70.41 58.49) (width 0.25) (layer "F.Cu") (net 6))
 (segment (start 70.36 58.49) (end 70.37 58.5) (width 0.25) (layer "F.Cu") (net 6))
 (segment (start 70.41 58.49) (end 70.42 58.5) (width 0.25) (layer "F.Cu") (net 6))
 (segment (start 65.659 58.4708) (end 64.3082 57.12) (width 0.25) (layer "F.Cu") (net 6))
 (segment (start 70.31 58.49) (end 70.32 58.5) (width 0.25) (layer "F.Cu") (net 6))
 (segment (start 64.3082 57.12) (end 61.62 57.12) (width 0.25) (layer "F.Cu") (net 6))
 (via (at 68.453 58.49) (size 0.6) (drill 0.3) (layers "F.Cu" "B.Cu") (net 6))
 (via (at 65.659 58.4708) (size 0.6) (drill 0.3) (layers "F.Cu" "B.Cu") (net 6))
 (segment (start 68.453 58.49) (end 65.6782 58.49) (width 0.25) (layer "B.Cu") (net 6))
 (segment (start 65.6782 58.49) (end 65.659 58.4708) (width 0.25) (layer "B.Cu") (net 6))
 (segment (start 59.7916 57.2008) (end 59.7408 57.2008) (width 0.25) (layer "F.Cu") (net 5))
 (segment (start 68.472931 59.517669) (end 70.402331 59.517669) (width 0.25) (layer "F.Cu") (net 5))
 (segment (start 68.472931 59.517669) (end 68.4906 59.5) (width 0.25) (layer "F.Cu") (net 5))
 (segment (start 70.402331 59.517669) (end 70.42 59.5) (width 0.25) (layer "F.Cu") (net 5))
 (segment (start 59.7408 57.2008) (end 56.4416 60.5) (width 0.25) (layer "F.Cu") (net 5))
 (segment (start 56.4416 60.5) (end 54.98 60.5) (width 0.25) (layer "F.Cu") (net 5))
 (segment (start 68.472931 59.517669) (end 68.455262 59.5) (width 0.25) (layer "F.Cu") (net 5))
 (segment (start 70.352331 59.517669) (end 70.37 59.5) (width 0.25) (layer "F.Cu") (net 5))
 (via (at 59.7916 57.2008) (size 0.6) (drill 0.3) (layers "F.Cu" "B.Cu") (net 5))
 (via (at 68.472931 59.517669) (size 0.6) (drill 0.3) (layers "F.Cu" "B.Cu") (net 5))
 (segment (start 61.4492 57.2008) (end 59.7916 57.2008) (width 0.25) (layer "B.Cu") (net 5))
 (segment (start 68.472931 59.517669) (end 65.791469 59.517669) (width 0.25) (layer "B.Cu") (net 5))
 (segment (start 65.791469 59.517669) (end 63.4638 57.19) (width 0.25) (layer "B.Cu") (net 5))
 (segment (start 61.46 57.19) (end 61.4492 57.2008) (width 0.25) (layer "B.Cu") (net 5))
 (segment (start 63.4638 57.19) (end 61.46 57.19) (width 0.25) (layer "B.Cu") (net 5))
 (segment (start 63.627 54.4068) (end 63.1698 54.864) (width 0.25) (layer "F.Cu") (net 9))
 (segment (start 64.5202 65.881) (end 64.5202 66.081) (width 0.25) (layer "F.Cu") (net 9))
 (segment (start 62.8402 65.941) (end 62.8452 65.936) (width 0.25) (layer "F.Cu") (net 9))
 (segment (start 63.5452 65.936) (end 64.4652 65.936) (width 0.25) (layer "F.Cu") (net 9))
 (segment (start 61.6202 65.941) (end 60.4038 65.941) (width 0.25) (layer "F.Cu") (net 9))
 (segment (start 65.6082 68.5546) (end 65.1502 68.0966) (width 0.25) (layer "F.Cu") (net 9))
 (segment (start 58.55 65.1) (end 58.55 65.5858) (width 0.25) (layer "F.Cu") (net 9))
 (segment (start 62.8452 65.936) (end 63.5452 65.936) (width 0.25) (layer "F.Cu") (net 9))
 (segment (start 61.727 52.847) (end 62.1942 52.847) (width 0.25) (layer "F.Cu") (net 9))
 (segment (start 68.5546 68.5292) (end 65.6336 68.5292) (width 0.25) (layer "F.Cu") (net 9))
 (segment (start 65.1502 66.711) (end 65.1502 67.481) (width 0.25) (layer "F.Cu") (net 9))
 (segment (start 68.4754 54.6354) (end 68.83 54.99) (width 0.25) (layer "F.Cu") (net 9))
 (segment (start 63.627 53.497) (end 64.1396 53.497) (width 0.25) (layer "F.Cu") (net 9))
 (segment (start 65.278 54.6354) (end 68.4754 54.6354) (width 0.25) (layer "F.Cu") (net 9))
 (segment (start 62.1942 52.847) (end 62.8442 53.497) (width 0.25) (layer "F.Cu") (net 9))
 (segment (start 64.5202 66.081) (end 65.1502 66.711) (width 0.25) (layer "F.Cu") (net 9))
 (segment (start 61.6202 65.941) (end 62.8402 65.941) (width 0.25) (layer "F.Cu") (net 9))
 (segment (start 59.5628 65.1) (end 58.55 65.1) (width 0.25) (layer "F.Cu") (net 9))
 (segment (start 65.6336 68.5292) (end 65.6082 68.5546) (width 0.25) (layer "F.Cu") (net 9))
 (segment (start 63.627 53.497) (end 63.627 54.4068) (width 0.25) (layer "F.Cu") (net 9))
 (segment (start 64.1396 53.497) (end 65.278 54.6354) (width 0.25) (layer "F.Cu") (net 9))
 (segment (start 69.9008 67.183) (end 68.5546 68.5292) (width 0.25) (layer "F.Cu") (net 9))
 (segment (start 60.4038 65.941) (end 59.5628 65.1) (width 0.25) (layer "F.Cu") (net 9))
 (segment (start 69.9008 63.881) (end 69.9008 67.183) (width 0.25) (layer "F.Cu") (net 9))
 (segment (start 62.8442 53.497) (end 63.627 53.497) (width 0.25) (layer "F.Cu") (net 9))
 (segment (start 65.1502 68.0966) (end 65.1502 67.481) (width 0.25) (layer "F.Cu") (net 9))
 (segment (start 64.4652 65.936) (end 64.5202 65.881) (width 0.25) (layer "F.Cu") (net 9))
 (via (at 69.9008 63.881) (size 0.6) (drill 0.3) (layers "F.Cu" "B.Cu") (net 9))
 (via (at 68.83 54.99) (size 0.6) (drill 0.3) (layers "F.Cu" "B.Cu") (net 9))
 (segment (start 69.9008 56.0832) (end 68.83 55.0124) (width 0.25) (layer "B.Cu") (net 9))
 (segment (start 68.83 55.0124) (end 68.83 54.99) (width 0.25) (layer "B.Cu") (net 9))
 (segment (start 69.9008 63.881) (end 69.9008 56.0832) (width 0.25) (layer "B.Cu") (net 9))
 (segment (start 68.426 63.981) (end 68.4276 63.9826) (width 0.25) (layer "F.Cu") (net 1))
 (segment (start 66.802 61.9252) (end 66.802 63.3476) (width 0.25) (layer "F.Cu") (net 1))
 (segment (start 62.7 59.2125) (end 64.0893 59.2125) (width 0.25) (layer "F.Cu") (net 1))
 (segment (start 66.7952 63.981) (end 68.426 63.981) (width 0.25) (layer "F.Cu") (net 1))
 (segment (start 64.0893 59.2125) (end 66.802 61.9252) (width 0.25) (layer "F.Cu") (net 1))
 (segment (start 66.7952 63.3544) (end 66.7952 63.981) (width 0.25) (layer "F.Cu") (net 1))
 (segment (start 66.802 63.3476) (end 66.7952 63.3544) (width 0.25) (layer "F.Cu") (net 1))
 (segment (start 60.0375 60.7875) (end 62.7 60.7875) (width 0.25) (layer "F.Cu") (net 2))
 (segment (start 57.6 63.225) (end 57.6 62.56) (width 0.25) (layer "F.Cu") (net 2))
 (segment (start 57.6 63.225) (end 60.0375 60.7875) (width 0.25) (layer "F.Cu") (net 2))
 (segment (start 62.0058 63.225) (end 59.5 63.225) (width 0.25) (layer "F.Cu") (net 8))
 (segment (start 59.545 63.18) (end 59.5 63.225) (width 0.25) (layer "F.Cu") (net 8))
 (segment (start 64.5202 63.981) (end 62.7618 63.981) (width 0.25) (layer "F.Cu") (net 8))
 (segment (start 62.7618 63.981) (end 62.0058 63.225) (width 0.25) (layer "F.Cu") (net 8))
 (segment (start 66.7952 67.346) (end 66.6602 67.481) (width 0.25) (layer "F.Cu") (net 7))
 (segment (start 67.7164 67.3608) (end 68.4276 67.3608) (width 0.25) (layer "F.Cu") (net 7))
 (segment (start 66.7952 65.881) (end 66.7952 67.196) (width 0.25) (layer "F.Cu") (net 7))
 (segment (start 66.5226 67.481) (end 67.5962 67.481) (width 0.25) (layer "F.Cu") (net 7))
 (segment (start 66.5226 67.481) (end 66.1702 67.481) (width 0.25) (layer "F.Cu") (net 7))
 (segment (start 66.7952 67.196) (end 66.7952 67.346) (width 0.25) (layer "F.Cu") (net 7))
 (segment (start 66.6602 67.481) (end 66.5226 67.481) (width 0.25) (layer "F.Cu") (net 7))
 (segment (start 67.5962 67.481) (end 67.7164 67.3608) (width 0.25) (layer "F.Cu") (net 7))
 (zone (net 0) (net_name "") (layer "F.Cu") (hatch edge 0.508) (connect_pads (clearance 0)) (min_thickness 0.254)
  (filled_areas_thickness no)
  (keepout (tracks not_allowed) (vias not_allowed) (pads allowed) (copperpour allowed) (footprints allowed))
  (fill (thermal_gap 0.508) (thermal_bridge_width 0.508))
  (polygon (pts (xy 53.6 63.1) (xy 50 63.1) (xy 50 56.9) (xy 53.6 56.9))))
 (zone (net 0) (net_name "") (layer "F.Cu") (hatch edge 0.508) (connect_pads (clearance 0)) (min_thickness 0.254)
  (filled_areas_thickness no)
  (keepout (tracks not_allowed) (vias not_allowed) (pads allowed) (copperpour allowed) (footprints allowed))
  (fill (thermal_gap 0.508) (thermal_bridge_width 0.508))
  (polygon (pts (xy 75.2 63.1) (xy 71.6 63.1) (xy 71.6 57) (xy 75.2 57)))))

